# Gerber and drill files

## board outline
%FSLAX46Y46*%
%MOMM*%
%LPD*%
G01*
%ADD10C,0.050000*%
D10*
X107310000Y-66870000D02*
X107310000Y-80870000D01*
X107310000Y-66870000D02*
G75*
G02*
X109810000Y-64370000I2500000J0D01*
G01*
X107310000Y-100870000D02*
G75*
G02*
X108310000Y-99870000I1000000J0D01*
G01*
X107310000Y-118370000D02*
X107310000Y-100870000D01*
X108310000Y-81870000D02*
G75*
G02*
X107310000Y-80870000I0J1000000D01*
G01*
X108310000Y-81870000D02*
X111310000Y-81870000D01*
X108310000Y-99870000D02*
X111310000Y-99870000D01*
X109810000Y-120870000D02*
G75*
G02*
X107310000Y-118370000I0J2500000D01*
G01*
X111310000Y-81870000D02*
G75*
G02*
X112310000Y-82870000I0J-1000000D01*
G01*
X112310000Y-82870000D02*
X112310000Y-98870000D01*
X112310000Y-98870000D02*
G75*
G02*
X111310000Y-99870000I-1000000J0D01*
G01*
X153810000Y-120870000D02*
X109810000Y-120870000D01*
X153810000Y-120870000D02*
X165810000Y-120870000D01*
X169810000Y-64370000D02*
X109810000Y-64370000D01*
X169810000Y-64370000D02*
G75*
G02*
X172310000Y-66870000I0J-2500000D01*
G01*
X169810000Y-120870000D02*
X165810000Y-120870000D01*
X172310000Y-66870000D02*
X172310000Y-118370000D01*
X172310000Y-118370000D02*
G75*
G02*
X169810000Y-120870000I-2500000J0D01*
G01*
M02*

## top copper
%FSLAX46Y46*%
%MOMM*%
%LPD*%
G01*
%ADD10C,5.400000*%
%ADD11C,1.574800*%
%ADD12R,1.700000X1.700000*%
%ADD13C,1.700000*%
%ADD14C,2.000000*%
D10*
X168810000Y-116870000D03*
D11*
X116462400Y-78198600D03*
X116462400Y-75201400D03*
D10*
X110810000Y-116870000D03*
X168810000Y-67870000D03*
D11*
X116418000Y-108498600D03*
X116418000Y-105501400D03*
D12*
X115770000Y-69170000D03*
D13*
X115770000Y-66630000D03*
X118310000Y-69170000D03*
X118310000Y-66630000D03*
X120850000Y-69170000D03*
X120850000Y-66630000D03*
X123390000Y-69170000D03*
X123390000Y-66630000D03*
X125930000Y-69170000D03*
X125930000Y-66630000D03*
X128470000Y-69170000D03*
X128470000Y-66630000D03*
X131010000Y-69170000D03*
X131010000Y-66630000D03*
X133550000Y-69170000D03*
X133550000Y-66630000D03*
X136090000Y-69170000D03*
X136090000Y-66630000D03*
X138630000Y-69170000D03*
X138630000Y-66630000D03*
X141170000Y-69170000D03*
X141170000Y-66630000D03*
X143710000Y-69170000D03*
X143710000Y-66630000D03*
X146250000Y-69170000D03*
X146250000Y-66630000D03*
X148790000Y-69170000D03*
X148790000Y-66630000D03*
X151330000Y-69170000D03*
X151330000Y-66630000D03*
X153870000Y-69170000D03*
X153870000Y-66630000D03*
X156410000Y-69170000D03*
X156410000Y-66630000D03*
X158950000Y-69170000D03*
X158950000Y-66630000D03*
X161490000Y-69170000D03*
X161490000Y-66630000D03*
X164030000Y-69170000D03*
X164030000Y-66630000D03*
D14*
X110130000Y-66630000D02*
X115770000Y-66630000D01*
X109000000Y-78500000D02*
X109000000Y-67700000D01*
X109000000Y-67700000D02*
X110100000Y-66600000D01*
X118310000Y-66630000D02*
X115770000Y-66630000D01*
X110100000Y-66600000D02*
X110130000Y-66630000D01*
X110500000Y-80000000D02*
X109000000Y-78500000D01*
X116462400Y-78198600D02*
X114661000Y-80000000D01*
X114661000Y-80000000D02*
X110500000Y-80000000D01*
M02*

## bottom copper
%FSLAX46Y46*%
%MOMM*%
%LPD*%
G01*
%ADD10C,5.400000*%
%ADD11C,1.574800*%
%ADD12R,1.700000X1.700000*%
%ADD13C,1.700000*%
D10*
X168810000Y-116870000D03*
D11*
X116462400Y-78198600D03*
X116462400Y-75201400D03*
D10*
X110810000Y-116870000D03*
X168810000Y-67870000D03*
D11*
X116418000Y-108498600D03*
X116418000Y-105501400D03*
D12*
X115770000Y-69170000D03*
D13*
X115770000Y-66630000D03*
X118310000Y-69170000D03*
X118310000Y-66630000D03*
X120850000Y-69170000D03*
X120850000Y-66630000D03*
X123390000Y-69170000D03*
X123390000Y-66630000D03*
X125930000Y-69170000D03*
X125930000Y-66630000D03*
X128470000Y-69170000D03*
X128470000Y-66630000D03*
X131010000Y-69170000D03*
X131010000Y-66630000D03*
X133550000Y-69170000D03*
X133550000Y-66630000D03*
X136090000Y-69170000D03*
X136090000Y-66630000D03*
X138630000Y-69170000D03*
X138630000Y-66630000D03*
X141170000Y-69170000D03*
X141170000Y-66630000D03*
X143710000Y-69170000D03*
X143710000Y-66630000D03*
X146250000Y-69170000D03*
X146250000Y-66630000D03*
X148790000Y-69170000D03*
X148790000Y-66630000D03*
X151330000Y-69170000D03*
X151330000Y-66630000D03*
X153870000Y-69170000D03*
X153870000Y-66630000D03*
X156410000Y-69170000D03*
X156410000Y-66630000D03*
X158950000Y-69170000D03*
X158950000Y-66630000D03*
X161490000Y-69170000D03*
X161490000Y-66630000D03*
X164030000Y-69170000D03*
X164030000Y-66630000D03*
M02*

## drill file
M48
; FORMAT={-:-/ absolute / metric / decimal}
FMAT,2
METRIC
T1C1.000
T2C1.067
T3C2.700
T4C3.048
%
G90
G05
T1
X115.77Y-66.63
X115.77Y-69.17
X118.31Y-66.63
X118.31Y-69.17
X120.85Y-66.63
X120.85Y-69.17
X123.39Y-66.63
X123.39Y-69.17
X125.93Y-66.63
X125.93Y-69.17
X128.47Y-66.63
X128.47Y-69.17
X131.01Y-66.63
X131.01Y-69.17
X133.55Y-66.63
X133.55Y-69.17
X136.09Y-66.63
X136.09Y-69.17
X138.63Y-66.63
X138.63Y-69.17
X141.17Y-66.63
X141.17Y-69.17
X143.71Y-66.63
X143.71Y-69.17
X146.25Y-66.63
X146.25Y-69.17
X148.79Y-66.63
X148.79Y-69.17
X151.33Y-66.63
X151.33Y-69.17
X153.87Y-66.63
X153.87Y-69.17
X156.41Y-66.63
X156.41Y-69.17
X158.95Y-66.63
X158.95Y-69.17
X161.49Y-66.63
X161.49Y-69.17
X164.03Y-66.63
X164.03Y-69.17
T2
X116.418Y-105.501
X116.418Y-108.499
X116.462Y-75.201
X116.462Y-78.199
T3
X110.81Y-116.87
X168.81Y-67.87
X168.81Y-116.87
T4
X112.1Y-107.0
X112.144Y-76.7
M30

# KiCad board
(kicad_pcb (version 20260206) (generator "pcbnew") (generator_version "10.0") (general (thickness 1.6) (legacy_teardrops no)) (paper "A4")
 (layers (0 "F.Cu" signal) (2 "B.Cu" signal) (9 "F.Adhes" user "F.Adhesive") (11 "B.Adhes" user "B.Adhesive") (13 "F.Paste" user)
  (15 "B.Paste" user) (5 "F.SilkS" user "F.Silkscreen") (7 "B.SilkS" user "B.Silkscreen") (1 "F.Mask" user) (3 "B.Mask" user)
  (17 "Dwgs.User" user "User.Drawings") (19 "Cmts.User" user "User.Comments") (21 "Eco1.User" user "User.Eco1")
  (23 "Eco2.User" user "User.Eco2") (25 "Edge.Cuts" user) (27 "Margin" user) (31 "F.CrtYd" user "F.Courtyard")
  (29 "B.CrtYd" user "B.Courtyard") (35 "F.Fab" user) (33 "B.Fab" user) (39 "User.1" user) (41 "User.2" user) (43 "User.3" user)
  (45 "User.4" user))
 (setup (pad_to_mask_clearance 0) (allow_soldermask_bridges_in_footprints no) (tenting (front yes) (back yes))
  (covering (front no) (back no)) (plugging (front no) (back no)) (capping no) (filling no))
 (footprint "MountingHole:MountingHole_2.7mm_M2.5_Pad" (layer "F.Cu") (at 168.81 116.87)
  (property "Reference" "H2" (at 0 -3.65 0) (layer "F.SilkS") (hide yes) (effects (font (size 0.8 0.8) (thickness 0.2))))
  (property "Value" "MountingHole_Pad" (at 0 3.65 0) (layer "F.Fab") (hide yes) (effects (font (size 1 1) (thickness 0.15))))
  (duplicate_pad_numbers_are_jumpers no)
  (pad "1" thru_hole circle (at 0 0) (size 5.4 5.4) (drill 2.7) (layers "*.Cu" "*.Mask") (remove_unused_layers no)
   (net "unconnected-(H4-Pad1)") (zone_connect 2)))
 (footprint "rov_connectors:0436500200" (layer "F.Cu") (at 116.4624 78.1986 -90)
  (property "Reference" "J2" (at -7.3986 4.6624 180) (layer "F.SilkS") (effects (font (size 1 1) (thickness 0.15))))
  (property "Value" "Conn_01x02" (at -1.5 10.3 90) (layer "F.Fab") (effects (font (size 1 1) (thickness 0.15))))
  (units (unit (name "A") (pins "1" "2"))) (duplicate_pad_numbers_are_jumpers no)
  (pad "" np_thru_hole circle (at -1.4986 4.318 270) (size 3.048 3.048) (drill 3.048) (layers "*.Cu" "*.Mask"))
  (pad "1" thru_hole circle (at 0 0 270) (size 1.5748 1.5748) (drill 1.0668) (layers "*.Cu" "*.Mask") (remove_unused_layers no)
   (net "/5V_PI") (solder_mask_margin 0.102))
  (pad "2" thru_hole circle (at -2.9972 0 270) (size 1.5748 1.5748) (drill 1.0668) (layers "*.Cu" "*.Mask") (remove_unused_layers no)
   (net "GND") (solder_mask_margin 0.102)))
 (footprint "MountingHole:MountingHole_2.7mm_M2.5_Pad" (layer "F.Cu") (at 110.81 116.87)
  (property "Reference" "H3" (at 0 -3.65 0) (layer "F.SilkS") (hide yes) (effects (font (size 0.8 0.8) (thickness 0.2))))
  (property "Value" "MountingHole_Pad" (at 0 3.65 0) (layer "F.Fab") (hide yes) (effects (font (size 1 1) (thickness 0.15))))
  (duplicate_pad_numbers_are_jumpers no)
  (pad "1" thru_hole circle (at 0 0) (size 5.4 5.4) (drill 2.7) (layers "*.Cu" "*.Mask") (remove_unused_layers no)
   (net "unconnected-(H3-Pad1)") (zone_connect 2)))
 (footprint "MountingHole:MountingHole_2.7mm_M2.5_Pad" (layer "F.Cu") (at 168.81 67.87)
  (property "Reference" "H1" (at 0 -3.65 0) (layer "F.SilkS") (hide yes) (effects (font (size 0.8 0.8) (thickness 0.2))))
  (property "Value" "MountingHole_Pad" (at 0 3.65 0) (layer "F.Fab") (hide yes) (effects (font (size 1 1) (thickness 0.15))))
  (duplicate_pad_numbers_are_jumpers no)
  (pad "1" thru_hole circle (at 0 0) (size 5.4 5.4) (drill 2.7) (layers "*.Cu" "*.Mask") (remove_unused_layers no)
   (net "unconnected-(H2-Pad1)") (zone_connect 2)))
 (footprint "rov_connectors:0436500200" (layer "F.Cu") (at 116.418 108.4986 -90)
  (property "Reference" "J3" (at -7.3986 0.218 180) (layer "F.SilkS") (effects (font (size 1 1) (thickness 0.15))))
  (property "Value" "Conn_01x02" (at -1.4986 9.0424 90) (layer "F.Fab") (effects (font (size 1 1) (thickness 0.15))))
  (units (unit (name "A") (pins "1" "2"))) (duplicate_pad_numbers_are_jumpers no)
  (pad "" np_thru_hole circle (at -1.4986 4.318 270) (size 3.048 3.048) (drill 3.048) (layers "*.Cu" "*.Mask"))
  (pad "1" thru_hole circle (at 0 0 270) (size 1.5748 1.5748) (drill 1.0668) (layers "*.Cu" "*.Mask") (remove_unused_layers no)
   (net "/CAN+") (solder_mask_margin 0.102))
  (pad "2" thru_hole circle (at -2.9972 0 270) (size 1.5748 1.5748) (drill 1.0668) (layers "*.Cu" "*.Mask") (remove_unused_layers no)
   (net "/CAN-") (solder_mask_margin 0.102)))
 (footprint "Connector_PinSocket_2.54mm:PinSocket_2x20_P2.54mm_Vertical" (layer "B.Cu") (at 115.77 69.17 -90)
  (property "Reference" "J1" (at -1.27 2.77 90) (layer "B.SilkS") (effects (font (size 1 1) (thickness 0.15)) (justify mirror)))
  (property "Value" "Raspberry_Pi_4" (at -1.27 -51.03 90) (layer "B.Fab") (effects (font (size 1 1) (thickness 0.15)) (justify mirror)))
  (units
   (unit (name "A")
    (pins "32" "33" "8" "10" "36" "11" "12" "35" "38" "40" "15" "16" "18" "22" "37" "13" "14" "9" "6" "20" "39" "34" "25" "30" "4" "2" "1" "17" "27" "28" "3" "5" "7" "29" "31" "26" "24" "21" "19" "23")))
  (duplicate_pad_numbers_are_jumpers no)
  (pad "1" thru_hole rect (at 0 0 270) (size 1.7 1.7) (drill 1) (layers "*.Cu" "*.Mask") (remove_unused_layers no) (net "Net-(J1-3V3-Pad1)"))
  (pad "2" thru_hole circle (at -2.54 0 270) (size 1.7 1.7) (drill 1) (layers "*.Cu" "*.Mask") (remove_unused_layers no) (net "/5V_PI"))
  (pad "3" thru_hole circle (at 0 -2.54 270) (size 1.7 1.7) (drill 1) (layers "*.Cu" "*.Mask") (remove_unused_layers no)
   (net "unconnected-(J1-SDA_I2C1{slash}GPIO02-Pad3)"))
  (pad "4" thru_hole circle (at -2.54 -2.54 270) (size 1.7 1.7) (drill 1) (layers "*.Cu" "*.Mask") (remove_unused_layers no) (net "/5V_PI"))
  (pad "5" thru_hole circle (at 0 -5.08 270) (size 1.7 1.7) (drill 1) (layers "*.Cu" "*.Mask") (remove_unused_layers no)
   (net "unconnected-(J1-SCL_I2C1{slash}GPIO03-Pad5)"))
  (pad "6" thru_hole circle (at -2.54 -5.08 270) (size 1.7 1.7) (drill 1) (layers "*.Cu" "*.Mask") (remove_unused_layers no) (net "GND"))
  (pad "7" thru_hole circle (at 0 -7.62 270) (size 1.7 1.7) (drill 1) (layers "*.Cu" "*.Mask") (remove_unused_layers no)
   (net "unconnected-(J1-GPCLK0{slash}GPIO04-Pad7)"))
  (pad "8" thru_hole circle (at -2.54 -7.62 270) (size 1.7 1.7) (drill 1) (layers "*.Cu" "*.Mask") (remove_unused_layers no) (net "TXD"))
  (pad "9" thru_hole circle (at 0 -10.16 270) (size 1.7 1.7) (drill 1) (layers "*.Cu" "*.Mask") (remove_unused_layers no) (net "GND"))
  (pad "10" thru_hole circle (at -2.54 -10.16 270) (size 1.7 1.7) (drill 1) (layers "*.Cu" "*.Mask") (remove_unused_layers no) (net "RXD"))
  (pad "11" thru_hole circle (at 0 -12.7 270) (size 1.7 1.7) (drill 1) (layers "*.Cu" "*.Mask") (remove_unused_layers no)
   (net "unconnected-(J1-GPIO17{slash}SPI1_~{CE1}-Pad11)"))
  (pad "12" thru_hole circle (at -2.54 -12.7 270) (size 1.7 1.7) (drill 1) (layers "*.Cu" "*.Mask") (remove_unused_layers no) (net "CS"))
  (pad "13" thru_hole circle (at 0 -15.24 270) (size 1.7 1.7) (drill 1) (layers "*.Cu" "*.Mask") (remove_unused_layers no)
   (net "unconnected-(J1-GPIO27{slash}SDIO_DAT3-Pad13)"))
  (pad "14" thru_hole circle (at -2.54 -15.24 270) (size 1.7 1.7) (drill 1) (layers "*.Cu" "*.Mask") (remove_unused_layers no) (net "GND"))
  (pad "15" thru_hole circle (at 0 -17.78 270) (size 1.7 1.7) (drill 1) (layers "*.Cu" "*.Mask") (remove_unused_layers no)
   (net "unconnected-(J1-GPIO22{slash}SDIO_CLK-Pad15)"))
  (pad "16" thru_hole circle (at -2.54 -17.78 270) (size 1.7 1.7) (drill 1) (layers "*.Cu" "*.Mask") (remove_unused_layers no)
   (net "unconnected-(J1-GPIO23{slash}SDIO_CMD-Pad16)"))
  (pad "17" thru_hole circle (at 0 -20.32 270) (size 1.7 1.7) (drill 1) (layers "*.Cu" "*.Mask") (remove_unused_layers no)
   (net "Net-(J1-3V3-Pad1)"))
  (pad "18" thru_hole circle (at -2.54 -20.32 270) (size 1.7 1.7) (drill 1) (layers "*.Cu" "*.Mask") (remove_unused_layers no)
   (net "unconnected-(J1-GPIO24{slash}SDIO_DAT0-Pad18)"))
  (pad "19" thru_hole circle (at 0 -22.86 270) (size 1.7 1.7) (drill 1) (layers "*.Cu" "*.Mask") (remove_unused_layers no)
   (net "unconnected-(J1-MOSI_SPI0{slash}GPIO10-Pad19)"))
  (pad "20" thru_hole circle (at -2.54 -22.86 270) (size 1.7 1.7) (drill 1) (layers "*.Cu" "*.Mask") (remove_unused_layers no) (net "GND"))
  (pad "21" thru_hole circle (at 0 -25.4 270) (size 1.7 1.7) (drill 1) (layers "*.Cu" "*.Mask") (remove_unused_layers no)
   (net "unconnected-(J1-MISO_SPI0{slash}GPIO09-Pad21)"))
  (pad "22" thru_hole circle (at -2.54 -25.4 270) (size 1.7 1.7) (drill 1) (layers "*.Cu" "*.Mask") (remove_unused_layers no)
   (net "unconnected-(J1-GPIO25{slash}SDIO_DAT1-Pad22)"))
  (pad "23" thru_hole circle (at 0 -27.94 270) (size 1.7 1.7) (drill 1) (layers "*.Cu" "*.Mask") (remove_unused_layers no)
   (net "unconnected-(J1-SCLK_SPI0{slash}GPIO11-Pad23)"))
  (pad "24" thru_hole circle (at -2.54 -27.94 270) (size 1.7 1.7) (drill 1) (layers "*.Cu" "*.Mask") (remove_unused_layers no)
   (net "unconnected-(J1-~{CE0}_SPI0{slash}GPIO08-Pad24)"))
  (pad "25" thru_hole circle (at 0 -30.48 270) (size 1.7 1.7) (drill 1) (layers "*.Cu" "*.Mask") (remove_unused_layers no) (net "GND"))
  (pad "26" thru_hole circle (at -2.54 -30.48 270) (size 1.7 1.7) (drill 1) (layers "*.Cu" "*.Mask") (remove_unused_layers no)
   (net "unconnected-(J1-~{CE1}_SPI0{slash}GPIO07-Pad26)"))
  (pad "27" thru_hole circle (at 0 -33.02 270) (size 1.7 1.7) (drill 1) (layers "*.Cu" "*.Mask") (remove_unused_layers no) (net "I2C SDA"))
  (pad "28" thru_hole circle (at -2.54 -33.02 270) (size 1.7 1.7) (drill 1) (layers "*.Cu" "*.Mask") (remove_unused_layers no)
   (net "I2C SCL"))
  (pad "29" thru_hole circle (at 0 -35.56 270) (size 1.7 1.7) (drill 1) (layers "*.Cu" "*.Mask") (remove_unused_layers no)
   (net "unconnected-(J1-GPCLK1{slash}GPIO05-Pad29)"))
  (pad "30" thru_hole circle (at -2.54 -35.56 270) (size 1.7 1.7) (drill 1) (layers "*.Cu" "*.Mask") (remove_unused_layers no) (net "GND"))
  (pad "31" thru_hole circle (at 0 -38.1 270) (size 1.7 1.7) (drill 1) (layers "*.Cu" "*.Mask") (remove_unused_layers no)
   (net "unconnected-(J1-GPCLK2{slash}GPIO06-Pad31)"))
  (pad "32" thru_hole circle (at -2.54 -38.1 270) (size 1.7 1.7) (drill 1) (layers "*.Cu" "*.Mask") (remove_unused_layers no)
   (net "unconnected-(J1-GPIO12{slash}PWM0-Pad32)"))
  (pad "33" thru_hole circle (at 0 -40.64 270) (size 1.7 1.7) (drill 1) (layers "*.Cu" "*.Mask") (remove_unused_layers no)
   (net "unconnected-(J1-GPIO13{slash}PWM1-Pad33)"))
  (pad "34" thru_hole circle (at -2.54 -40.64 270) (size 1.7 1.7) (drill 1) (layers "*.Cu" "*.Mask") (remove_unused_layers no) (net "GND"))
  (pad "35" thru_hole circle (at 0 -43.18 270) (size 1.7 1.7) (drill 1) (layers "*.Cu" "*.Mask") (remove_unused_layers no) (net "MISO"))
  (pad "36" thru_hole circle (at -2.54 -43.18 270) (size 1.7 1.7) (drill 1) (layers "*.Cu" "*.Mask") (remove_unused_layers no)
   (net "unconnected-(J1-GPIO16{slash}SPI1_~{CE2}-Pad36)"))
  (pad "37" thru_hole circle (at 0 -45.72 270) (size 1.7 1.7) (drill 1) (layers "*.Cu" "*.Mask") (remove_unused_layers no)
   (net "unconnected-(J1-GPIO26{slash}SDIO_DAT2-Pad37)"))
  (pad "38" thru_hole circle (at -2.54 -45.72 270) (size 1.7 1.7) (drill 1) (layers "*.Cu" "*.Mask") (remove_unused_layers no) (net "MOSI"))
  (pad "39" thru_hole circle (at 0 -48.26 270) (size 1.7 1.7) (drill 1) (layers "*.Cu" "*.Mask") (remove_unused_layers no) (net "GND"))
  (pad "40" thru_hole circle (at -2.54 -48.26 270) (size 1.7 1.7) (drill 1) (layers "*.Cu" "*.Mask") (remove_unused_layers no) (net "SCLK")))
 (gr_line (start 107.31 66.87) (end 107.31 80.87) (stroke (width 0.05) (type solid)) (layer "Edge.Cuts"))
 (gr_arc (start 107.31 66.87) (mid 108.042233 65.102233) (end 109.81 64.37) (stroke (width 0.05) (type default)) (layer "Edge.Cuts"))
 (gr_arc (start 107.31 100.87) (mid 107.602893 100.162893) (end 108.31 99.87) (stroke (width 0.05) (type default)) (layer "Edge.Cuts"))
 (gr_line (start 107.31 118.37) (end 107.31 100.87) (stroke (width 0.05) (type solid)) (layer "Edge.Cuts"))
 (gr_arc (start 108.31 81.87) (mid 107.602893 81.577107) (end 107.31 80.87) (stroke (width 0.05) (type default)) (layer "Edge.Cuts"))
 (gr_line (start 108.31 81.87) (end 111.31 81.87) (stroke (width 0.05) (type solid)) (layer "Edge.Cuts"))
 (gr_line (start 108.31 99.87) (end 111.31 99.87) (stroke (width 0.05) (type solid)) (layer "Edge.Cuts"))
 (gr_arc (start 109.81 120.87) (mid 108.042233 120.137767) (end 107.31 118.37) (stroke (width 0.05) (type default)) (layer "Edge.Cuts"))
 (gr_arc (start 111.31 81.87) (mid 112.017107 82.162893) (end 112.31 82.87) (stroke (width 0.05) (type default)) (layer "Edge.Cuts"))
 (gr_line (start 112.31 82.87) (end 112.31 98.87) (stroke (width 0.05) (type default)) (layer "Edge.Cuts"))
 (gr_arc (start 112.31 98.87) (mid 112.017107 99.577107) (end 111.31 99.87) (stroke (width 0.05) (type default)) (layer "Edge.Cuts"))
 (gr_line (start 153.81 120.87) (end 109.81 120.87) (stroke (width 0.05) (type solid)) (layer "Edge.Cuts"))
 (gr_line (start 153.81 120.87) (end 165.81 120.87) (stroke (width 0.05) (type default)) (layer "Edge.Cuts"))
 (gr_line (start 169.81 64.37) (end 109.81 64.37) (stroke (width 0.05) (type solid)) (layer "Edge.Cuts"))
 (gr_arc (start 169.81 64.37) (mid 171.577767 65.102233) (end 172.31 66.87) (stroke (width 0.05) (type default)) (layer "Edge.Cuts"))
 (gr_line (start 169.81 120.87) (end 165.81 120.87) (stroke (width 0.05) (type solid)) (layer "Edge.Cuts"))
 (gr_line (start 172.31 66.87) (end 172.31 118.37) (stroke (width 0.05) (type solid)) (layer "Edge.Cuts"))
 (gr_arc (start 172.31 118.37) (mid 171.577767 120.137767) (end 169.81 120.87) (stroke (width 0.05) (type default)) (layer "Edge.Cuts"))
 (segment (start 110.13 66.63) (end 115.77 66.63) (width 2) (layer "F.Cu") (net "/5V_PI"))
 (segment (start 109 78.5) (end 109 67.7) (width 2) (layer "F.Cu") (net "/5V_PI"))
 (segment (start 109 67.7) (end 110.1 66.6) (width 2) (layer "F.Cu") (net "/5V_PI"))
 (segment (start 118.31 66.63) (end 115.77 66.63) (width 2) (layer "F.Cu") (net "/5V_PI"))
 (segment (start 110.1 66.6) (end 110.13 66.63) (width 2) (layer "F.Cu") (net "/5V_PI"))
 (segment (start 110.5 80) (end 109 78.5) (width 2) (layer "F.Cu") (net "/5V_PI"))
 (segment (start 116.4624 78.1986) (end 114.661 80) (width 2) (layer "F.Cu") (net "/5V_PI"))
 (segment (start 114.661 80) (end 110.5 80) (width 2) (layer "F.Cu") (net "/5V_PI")))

